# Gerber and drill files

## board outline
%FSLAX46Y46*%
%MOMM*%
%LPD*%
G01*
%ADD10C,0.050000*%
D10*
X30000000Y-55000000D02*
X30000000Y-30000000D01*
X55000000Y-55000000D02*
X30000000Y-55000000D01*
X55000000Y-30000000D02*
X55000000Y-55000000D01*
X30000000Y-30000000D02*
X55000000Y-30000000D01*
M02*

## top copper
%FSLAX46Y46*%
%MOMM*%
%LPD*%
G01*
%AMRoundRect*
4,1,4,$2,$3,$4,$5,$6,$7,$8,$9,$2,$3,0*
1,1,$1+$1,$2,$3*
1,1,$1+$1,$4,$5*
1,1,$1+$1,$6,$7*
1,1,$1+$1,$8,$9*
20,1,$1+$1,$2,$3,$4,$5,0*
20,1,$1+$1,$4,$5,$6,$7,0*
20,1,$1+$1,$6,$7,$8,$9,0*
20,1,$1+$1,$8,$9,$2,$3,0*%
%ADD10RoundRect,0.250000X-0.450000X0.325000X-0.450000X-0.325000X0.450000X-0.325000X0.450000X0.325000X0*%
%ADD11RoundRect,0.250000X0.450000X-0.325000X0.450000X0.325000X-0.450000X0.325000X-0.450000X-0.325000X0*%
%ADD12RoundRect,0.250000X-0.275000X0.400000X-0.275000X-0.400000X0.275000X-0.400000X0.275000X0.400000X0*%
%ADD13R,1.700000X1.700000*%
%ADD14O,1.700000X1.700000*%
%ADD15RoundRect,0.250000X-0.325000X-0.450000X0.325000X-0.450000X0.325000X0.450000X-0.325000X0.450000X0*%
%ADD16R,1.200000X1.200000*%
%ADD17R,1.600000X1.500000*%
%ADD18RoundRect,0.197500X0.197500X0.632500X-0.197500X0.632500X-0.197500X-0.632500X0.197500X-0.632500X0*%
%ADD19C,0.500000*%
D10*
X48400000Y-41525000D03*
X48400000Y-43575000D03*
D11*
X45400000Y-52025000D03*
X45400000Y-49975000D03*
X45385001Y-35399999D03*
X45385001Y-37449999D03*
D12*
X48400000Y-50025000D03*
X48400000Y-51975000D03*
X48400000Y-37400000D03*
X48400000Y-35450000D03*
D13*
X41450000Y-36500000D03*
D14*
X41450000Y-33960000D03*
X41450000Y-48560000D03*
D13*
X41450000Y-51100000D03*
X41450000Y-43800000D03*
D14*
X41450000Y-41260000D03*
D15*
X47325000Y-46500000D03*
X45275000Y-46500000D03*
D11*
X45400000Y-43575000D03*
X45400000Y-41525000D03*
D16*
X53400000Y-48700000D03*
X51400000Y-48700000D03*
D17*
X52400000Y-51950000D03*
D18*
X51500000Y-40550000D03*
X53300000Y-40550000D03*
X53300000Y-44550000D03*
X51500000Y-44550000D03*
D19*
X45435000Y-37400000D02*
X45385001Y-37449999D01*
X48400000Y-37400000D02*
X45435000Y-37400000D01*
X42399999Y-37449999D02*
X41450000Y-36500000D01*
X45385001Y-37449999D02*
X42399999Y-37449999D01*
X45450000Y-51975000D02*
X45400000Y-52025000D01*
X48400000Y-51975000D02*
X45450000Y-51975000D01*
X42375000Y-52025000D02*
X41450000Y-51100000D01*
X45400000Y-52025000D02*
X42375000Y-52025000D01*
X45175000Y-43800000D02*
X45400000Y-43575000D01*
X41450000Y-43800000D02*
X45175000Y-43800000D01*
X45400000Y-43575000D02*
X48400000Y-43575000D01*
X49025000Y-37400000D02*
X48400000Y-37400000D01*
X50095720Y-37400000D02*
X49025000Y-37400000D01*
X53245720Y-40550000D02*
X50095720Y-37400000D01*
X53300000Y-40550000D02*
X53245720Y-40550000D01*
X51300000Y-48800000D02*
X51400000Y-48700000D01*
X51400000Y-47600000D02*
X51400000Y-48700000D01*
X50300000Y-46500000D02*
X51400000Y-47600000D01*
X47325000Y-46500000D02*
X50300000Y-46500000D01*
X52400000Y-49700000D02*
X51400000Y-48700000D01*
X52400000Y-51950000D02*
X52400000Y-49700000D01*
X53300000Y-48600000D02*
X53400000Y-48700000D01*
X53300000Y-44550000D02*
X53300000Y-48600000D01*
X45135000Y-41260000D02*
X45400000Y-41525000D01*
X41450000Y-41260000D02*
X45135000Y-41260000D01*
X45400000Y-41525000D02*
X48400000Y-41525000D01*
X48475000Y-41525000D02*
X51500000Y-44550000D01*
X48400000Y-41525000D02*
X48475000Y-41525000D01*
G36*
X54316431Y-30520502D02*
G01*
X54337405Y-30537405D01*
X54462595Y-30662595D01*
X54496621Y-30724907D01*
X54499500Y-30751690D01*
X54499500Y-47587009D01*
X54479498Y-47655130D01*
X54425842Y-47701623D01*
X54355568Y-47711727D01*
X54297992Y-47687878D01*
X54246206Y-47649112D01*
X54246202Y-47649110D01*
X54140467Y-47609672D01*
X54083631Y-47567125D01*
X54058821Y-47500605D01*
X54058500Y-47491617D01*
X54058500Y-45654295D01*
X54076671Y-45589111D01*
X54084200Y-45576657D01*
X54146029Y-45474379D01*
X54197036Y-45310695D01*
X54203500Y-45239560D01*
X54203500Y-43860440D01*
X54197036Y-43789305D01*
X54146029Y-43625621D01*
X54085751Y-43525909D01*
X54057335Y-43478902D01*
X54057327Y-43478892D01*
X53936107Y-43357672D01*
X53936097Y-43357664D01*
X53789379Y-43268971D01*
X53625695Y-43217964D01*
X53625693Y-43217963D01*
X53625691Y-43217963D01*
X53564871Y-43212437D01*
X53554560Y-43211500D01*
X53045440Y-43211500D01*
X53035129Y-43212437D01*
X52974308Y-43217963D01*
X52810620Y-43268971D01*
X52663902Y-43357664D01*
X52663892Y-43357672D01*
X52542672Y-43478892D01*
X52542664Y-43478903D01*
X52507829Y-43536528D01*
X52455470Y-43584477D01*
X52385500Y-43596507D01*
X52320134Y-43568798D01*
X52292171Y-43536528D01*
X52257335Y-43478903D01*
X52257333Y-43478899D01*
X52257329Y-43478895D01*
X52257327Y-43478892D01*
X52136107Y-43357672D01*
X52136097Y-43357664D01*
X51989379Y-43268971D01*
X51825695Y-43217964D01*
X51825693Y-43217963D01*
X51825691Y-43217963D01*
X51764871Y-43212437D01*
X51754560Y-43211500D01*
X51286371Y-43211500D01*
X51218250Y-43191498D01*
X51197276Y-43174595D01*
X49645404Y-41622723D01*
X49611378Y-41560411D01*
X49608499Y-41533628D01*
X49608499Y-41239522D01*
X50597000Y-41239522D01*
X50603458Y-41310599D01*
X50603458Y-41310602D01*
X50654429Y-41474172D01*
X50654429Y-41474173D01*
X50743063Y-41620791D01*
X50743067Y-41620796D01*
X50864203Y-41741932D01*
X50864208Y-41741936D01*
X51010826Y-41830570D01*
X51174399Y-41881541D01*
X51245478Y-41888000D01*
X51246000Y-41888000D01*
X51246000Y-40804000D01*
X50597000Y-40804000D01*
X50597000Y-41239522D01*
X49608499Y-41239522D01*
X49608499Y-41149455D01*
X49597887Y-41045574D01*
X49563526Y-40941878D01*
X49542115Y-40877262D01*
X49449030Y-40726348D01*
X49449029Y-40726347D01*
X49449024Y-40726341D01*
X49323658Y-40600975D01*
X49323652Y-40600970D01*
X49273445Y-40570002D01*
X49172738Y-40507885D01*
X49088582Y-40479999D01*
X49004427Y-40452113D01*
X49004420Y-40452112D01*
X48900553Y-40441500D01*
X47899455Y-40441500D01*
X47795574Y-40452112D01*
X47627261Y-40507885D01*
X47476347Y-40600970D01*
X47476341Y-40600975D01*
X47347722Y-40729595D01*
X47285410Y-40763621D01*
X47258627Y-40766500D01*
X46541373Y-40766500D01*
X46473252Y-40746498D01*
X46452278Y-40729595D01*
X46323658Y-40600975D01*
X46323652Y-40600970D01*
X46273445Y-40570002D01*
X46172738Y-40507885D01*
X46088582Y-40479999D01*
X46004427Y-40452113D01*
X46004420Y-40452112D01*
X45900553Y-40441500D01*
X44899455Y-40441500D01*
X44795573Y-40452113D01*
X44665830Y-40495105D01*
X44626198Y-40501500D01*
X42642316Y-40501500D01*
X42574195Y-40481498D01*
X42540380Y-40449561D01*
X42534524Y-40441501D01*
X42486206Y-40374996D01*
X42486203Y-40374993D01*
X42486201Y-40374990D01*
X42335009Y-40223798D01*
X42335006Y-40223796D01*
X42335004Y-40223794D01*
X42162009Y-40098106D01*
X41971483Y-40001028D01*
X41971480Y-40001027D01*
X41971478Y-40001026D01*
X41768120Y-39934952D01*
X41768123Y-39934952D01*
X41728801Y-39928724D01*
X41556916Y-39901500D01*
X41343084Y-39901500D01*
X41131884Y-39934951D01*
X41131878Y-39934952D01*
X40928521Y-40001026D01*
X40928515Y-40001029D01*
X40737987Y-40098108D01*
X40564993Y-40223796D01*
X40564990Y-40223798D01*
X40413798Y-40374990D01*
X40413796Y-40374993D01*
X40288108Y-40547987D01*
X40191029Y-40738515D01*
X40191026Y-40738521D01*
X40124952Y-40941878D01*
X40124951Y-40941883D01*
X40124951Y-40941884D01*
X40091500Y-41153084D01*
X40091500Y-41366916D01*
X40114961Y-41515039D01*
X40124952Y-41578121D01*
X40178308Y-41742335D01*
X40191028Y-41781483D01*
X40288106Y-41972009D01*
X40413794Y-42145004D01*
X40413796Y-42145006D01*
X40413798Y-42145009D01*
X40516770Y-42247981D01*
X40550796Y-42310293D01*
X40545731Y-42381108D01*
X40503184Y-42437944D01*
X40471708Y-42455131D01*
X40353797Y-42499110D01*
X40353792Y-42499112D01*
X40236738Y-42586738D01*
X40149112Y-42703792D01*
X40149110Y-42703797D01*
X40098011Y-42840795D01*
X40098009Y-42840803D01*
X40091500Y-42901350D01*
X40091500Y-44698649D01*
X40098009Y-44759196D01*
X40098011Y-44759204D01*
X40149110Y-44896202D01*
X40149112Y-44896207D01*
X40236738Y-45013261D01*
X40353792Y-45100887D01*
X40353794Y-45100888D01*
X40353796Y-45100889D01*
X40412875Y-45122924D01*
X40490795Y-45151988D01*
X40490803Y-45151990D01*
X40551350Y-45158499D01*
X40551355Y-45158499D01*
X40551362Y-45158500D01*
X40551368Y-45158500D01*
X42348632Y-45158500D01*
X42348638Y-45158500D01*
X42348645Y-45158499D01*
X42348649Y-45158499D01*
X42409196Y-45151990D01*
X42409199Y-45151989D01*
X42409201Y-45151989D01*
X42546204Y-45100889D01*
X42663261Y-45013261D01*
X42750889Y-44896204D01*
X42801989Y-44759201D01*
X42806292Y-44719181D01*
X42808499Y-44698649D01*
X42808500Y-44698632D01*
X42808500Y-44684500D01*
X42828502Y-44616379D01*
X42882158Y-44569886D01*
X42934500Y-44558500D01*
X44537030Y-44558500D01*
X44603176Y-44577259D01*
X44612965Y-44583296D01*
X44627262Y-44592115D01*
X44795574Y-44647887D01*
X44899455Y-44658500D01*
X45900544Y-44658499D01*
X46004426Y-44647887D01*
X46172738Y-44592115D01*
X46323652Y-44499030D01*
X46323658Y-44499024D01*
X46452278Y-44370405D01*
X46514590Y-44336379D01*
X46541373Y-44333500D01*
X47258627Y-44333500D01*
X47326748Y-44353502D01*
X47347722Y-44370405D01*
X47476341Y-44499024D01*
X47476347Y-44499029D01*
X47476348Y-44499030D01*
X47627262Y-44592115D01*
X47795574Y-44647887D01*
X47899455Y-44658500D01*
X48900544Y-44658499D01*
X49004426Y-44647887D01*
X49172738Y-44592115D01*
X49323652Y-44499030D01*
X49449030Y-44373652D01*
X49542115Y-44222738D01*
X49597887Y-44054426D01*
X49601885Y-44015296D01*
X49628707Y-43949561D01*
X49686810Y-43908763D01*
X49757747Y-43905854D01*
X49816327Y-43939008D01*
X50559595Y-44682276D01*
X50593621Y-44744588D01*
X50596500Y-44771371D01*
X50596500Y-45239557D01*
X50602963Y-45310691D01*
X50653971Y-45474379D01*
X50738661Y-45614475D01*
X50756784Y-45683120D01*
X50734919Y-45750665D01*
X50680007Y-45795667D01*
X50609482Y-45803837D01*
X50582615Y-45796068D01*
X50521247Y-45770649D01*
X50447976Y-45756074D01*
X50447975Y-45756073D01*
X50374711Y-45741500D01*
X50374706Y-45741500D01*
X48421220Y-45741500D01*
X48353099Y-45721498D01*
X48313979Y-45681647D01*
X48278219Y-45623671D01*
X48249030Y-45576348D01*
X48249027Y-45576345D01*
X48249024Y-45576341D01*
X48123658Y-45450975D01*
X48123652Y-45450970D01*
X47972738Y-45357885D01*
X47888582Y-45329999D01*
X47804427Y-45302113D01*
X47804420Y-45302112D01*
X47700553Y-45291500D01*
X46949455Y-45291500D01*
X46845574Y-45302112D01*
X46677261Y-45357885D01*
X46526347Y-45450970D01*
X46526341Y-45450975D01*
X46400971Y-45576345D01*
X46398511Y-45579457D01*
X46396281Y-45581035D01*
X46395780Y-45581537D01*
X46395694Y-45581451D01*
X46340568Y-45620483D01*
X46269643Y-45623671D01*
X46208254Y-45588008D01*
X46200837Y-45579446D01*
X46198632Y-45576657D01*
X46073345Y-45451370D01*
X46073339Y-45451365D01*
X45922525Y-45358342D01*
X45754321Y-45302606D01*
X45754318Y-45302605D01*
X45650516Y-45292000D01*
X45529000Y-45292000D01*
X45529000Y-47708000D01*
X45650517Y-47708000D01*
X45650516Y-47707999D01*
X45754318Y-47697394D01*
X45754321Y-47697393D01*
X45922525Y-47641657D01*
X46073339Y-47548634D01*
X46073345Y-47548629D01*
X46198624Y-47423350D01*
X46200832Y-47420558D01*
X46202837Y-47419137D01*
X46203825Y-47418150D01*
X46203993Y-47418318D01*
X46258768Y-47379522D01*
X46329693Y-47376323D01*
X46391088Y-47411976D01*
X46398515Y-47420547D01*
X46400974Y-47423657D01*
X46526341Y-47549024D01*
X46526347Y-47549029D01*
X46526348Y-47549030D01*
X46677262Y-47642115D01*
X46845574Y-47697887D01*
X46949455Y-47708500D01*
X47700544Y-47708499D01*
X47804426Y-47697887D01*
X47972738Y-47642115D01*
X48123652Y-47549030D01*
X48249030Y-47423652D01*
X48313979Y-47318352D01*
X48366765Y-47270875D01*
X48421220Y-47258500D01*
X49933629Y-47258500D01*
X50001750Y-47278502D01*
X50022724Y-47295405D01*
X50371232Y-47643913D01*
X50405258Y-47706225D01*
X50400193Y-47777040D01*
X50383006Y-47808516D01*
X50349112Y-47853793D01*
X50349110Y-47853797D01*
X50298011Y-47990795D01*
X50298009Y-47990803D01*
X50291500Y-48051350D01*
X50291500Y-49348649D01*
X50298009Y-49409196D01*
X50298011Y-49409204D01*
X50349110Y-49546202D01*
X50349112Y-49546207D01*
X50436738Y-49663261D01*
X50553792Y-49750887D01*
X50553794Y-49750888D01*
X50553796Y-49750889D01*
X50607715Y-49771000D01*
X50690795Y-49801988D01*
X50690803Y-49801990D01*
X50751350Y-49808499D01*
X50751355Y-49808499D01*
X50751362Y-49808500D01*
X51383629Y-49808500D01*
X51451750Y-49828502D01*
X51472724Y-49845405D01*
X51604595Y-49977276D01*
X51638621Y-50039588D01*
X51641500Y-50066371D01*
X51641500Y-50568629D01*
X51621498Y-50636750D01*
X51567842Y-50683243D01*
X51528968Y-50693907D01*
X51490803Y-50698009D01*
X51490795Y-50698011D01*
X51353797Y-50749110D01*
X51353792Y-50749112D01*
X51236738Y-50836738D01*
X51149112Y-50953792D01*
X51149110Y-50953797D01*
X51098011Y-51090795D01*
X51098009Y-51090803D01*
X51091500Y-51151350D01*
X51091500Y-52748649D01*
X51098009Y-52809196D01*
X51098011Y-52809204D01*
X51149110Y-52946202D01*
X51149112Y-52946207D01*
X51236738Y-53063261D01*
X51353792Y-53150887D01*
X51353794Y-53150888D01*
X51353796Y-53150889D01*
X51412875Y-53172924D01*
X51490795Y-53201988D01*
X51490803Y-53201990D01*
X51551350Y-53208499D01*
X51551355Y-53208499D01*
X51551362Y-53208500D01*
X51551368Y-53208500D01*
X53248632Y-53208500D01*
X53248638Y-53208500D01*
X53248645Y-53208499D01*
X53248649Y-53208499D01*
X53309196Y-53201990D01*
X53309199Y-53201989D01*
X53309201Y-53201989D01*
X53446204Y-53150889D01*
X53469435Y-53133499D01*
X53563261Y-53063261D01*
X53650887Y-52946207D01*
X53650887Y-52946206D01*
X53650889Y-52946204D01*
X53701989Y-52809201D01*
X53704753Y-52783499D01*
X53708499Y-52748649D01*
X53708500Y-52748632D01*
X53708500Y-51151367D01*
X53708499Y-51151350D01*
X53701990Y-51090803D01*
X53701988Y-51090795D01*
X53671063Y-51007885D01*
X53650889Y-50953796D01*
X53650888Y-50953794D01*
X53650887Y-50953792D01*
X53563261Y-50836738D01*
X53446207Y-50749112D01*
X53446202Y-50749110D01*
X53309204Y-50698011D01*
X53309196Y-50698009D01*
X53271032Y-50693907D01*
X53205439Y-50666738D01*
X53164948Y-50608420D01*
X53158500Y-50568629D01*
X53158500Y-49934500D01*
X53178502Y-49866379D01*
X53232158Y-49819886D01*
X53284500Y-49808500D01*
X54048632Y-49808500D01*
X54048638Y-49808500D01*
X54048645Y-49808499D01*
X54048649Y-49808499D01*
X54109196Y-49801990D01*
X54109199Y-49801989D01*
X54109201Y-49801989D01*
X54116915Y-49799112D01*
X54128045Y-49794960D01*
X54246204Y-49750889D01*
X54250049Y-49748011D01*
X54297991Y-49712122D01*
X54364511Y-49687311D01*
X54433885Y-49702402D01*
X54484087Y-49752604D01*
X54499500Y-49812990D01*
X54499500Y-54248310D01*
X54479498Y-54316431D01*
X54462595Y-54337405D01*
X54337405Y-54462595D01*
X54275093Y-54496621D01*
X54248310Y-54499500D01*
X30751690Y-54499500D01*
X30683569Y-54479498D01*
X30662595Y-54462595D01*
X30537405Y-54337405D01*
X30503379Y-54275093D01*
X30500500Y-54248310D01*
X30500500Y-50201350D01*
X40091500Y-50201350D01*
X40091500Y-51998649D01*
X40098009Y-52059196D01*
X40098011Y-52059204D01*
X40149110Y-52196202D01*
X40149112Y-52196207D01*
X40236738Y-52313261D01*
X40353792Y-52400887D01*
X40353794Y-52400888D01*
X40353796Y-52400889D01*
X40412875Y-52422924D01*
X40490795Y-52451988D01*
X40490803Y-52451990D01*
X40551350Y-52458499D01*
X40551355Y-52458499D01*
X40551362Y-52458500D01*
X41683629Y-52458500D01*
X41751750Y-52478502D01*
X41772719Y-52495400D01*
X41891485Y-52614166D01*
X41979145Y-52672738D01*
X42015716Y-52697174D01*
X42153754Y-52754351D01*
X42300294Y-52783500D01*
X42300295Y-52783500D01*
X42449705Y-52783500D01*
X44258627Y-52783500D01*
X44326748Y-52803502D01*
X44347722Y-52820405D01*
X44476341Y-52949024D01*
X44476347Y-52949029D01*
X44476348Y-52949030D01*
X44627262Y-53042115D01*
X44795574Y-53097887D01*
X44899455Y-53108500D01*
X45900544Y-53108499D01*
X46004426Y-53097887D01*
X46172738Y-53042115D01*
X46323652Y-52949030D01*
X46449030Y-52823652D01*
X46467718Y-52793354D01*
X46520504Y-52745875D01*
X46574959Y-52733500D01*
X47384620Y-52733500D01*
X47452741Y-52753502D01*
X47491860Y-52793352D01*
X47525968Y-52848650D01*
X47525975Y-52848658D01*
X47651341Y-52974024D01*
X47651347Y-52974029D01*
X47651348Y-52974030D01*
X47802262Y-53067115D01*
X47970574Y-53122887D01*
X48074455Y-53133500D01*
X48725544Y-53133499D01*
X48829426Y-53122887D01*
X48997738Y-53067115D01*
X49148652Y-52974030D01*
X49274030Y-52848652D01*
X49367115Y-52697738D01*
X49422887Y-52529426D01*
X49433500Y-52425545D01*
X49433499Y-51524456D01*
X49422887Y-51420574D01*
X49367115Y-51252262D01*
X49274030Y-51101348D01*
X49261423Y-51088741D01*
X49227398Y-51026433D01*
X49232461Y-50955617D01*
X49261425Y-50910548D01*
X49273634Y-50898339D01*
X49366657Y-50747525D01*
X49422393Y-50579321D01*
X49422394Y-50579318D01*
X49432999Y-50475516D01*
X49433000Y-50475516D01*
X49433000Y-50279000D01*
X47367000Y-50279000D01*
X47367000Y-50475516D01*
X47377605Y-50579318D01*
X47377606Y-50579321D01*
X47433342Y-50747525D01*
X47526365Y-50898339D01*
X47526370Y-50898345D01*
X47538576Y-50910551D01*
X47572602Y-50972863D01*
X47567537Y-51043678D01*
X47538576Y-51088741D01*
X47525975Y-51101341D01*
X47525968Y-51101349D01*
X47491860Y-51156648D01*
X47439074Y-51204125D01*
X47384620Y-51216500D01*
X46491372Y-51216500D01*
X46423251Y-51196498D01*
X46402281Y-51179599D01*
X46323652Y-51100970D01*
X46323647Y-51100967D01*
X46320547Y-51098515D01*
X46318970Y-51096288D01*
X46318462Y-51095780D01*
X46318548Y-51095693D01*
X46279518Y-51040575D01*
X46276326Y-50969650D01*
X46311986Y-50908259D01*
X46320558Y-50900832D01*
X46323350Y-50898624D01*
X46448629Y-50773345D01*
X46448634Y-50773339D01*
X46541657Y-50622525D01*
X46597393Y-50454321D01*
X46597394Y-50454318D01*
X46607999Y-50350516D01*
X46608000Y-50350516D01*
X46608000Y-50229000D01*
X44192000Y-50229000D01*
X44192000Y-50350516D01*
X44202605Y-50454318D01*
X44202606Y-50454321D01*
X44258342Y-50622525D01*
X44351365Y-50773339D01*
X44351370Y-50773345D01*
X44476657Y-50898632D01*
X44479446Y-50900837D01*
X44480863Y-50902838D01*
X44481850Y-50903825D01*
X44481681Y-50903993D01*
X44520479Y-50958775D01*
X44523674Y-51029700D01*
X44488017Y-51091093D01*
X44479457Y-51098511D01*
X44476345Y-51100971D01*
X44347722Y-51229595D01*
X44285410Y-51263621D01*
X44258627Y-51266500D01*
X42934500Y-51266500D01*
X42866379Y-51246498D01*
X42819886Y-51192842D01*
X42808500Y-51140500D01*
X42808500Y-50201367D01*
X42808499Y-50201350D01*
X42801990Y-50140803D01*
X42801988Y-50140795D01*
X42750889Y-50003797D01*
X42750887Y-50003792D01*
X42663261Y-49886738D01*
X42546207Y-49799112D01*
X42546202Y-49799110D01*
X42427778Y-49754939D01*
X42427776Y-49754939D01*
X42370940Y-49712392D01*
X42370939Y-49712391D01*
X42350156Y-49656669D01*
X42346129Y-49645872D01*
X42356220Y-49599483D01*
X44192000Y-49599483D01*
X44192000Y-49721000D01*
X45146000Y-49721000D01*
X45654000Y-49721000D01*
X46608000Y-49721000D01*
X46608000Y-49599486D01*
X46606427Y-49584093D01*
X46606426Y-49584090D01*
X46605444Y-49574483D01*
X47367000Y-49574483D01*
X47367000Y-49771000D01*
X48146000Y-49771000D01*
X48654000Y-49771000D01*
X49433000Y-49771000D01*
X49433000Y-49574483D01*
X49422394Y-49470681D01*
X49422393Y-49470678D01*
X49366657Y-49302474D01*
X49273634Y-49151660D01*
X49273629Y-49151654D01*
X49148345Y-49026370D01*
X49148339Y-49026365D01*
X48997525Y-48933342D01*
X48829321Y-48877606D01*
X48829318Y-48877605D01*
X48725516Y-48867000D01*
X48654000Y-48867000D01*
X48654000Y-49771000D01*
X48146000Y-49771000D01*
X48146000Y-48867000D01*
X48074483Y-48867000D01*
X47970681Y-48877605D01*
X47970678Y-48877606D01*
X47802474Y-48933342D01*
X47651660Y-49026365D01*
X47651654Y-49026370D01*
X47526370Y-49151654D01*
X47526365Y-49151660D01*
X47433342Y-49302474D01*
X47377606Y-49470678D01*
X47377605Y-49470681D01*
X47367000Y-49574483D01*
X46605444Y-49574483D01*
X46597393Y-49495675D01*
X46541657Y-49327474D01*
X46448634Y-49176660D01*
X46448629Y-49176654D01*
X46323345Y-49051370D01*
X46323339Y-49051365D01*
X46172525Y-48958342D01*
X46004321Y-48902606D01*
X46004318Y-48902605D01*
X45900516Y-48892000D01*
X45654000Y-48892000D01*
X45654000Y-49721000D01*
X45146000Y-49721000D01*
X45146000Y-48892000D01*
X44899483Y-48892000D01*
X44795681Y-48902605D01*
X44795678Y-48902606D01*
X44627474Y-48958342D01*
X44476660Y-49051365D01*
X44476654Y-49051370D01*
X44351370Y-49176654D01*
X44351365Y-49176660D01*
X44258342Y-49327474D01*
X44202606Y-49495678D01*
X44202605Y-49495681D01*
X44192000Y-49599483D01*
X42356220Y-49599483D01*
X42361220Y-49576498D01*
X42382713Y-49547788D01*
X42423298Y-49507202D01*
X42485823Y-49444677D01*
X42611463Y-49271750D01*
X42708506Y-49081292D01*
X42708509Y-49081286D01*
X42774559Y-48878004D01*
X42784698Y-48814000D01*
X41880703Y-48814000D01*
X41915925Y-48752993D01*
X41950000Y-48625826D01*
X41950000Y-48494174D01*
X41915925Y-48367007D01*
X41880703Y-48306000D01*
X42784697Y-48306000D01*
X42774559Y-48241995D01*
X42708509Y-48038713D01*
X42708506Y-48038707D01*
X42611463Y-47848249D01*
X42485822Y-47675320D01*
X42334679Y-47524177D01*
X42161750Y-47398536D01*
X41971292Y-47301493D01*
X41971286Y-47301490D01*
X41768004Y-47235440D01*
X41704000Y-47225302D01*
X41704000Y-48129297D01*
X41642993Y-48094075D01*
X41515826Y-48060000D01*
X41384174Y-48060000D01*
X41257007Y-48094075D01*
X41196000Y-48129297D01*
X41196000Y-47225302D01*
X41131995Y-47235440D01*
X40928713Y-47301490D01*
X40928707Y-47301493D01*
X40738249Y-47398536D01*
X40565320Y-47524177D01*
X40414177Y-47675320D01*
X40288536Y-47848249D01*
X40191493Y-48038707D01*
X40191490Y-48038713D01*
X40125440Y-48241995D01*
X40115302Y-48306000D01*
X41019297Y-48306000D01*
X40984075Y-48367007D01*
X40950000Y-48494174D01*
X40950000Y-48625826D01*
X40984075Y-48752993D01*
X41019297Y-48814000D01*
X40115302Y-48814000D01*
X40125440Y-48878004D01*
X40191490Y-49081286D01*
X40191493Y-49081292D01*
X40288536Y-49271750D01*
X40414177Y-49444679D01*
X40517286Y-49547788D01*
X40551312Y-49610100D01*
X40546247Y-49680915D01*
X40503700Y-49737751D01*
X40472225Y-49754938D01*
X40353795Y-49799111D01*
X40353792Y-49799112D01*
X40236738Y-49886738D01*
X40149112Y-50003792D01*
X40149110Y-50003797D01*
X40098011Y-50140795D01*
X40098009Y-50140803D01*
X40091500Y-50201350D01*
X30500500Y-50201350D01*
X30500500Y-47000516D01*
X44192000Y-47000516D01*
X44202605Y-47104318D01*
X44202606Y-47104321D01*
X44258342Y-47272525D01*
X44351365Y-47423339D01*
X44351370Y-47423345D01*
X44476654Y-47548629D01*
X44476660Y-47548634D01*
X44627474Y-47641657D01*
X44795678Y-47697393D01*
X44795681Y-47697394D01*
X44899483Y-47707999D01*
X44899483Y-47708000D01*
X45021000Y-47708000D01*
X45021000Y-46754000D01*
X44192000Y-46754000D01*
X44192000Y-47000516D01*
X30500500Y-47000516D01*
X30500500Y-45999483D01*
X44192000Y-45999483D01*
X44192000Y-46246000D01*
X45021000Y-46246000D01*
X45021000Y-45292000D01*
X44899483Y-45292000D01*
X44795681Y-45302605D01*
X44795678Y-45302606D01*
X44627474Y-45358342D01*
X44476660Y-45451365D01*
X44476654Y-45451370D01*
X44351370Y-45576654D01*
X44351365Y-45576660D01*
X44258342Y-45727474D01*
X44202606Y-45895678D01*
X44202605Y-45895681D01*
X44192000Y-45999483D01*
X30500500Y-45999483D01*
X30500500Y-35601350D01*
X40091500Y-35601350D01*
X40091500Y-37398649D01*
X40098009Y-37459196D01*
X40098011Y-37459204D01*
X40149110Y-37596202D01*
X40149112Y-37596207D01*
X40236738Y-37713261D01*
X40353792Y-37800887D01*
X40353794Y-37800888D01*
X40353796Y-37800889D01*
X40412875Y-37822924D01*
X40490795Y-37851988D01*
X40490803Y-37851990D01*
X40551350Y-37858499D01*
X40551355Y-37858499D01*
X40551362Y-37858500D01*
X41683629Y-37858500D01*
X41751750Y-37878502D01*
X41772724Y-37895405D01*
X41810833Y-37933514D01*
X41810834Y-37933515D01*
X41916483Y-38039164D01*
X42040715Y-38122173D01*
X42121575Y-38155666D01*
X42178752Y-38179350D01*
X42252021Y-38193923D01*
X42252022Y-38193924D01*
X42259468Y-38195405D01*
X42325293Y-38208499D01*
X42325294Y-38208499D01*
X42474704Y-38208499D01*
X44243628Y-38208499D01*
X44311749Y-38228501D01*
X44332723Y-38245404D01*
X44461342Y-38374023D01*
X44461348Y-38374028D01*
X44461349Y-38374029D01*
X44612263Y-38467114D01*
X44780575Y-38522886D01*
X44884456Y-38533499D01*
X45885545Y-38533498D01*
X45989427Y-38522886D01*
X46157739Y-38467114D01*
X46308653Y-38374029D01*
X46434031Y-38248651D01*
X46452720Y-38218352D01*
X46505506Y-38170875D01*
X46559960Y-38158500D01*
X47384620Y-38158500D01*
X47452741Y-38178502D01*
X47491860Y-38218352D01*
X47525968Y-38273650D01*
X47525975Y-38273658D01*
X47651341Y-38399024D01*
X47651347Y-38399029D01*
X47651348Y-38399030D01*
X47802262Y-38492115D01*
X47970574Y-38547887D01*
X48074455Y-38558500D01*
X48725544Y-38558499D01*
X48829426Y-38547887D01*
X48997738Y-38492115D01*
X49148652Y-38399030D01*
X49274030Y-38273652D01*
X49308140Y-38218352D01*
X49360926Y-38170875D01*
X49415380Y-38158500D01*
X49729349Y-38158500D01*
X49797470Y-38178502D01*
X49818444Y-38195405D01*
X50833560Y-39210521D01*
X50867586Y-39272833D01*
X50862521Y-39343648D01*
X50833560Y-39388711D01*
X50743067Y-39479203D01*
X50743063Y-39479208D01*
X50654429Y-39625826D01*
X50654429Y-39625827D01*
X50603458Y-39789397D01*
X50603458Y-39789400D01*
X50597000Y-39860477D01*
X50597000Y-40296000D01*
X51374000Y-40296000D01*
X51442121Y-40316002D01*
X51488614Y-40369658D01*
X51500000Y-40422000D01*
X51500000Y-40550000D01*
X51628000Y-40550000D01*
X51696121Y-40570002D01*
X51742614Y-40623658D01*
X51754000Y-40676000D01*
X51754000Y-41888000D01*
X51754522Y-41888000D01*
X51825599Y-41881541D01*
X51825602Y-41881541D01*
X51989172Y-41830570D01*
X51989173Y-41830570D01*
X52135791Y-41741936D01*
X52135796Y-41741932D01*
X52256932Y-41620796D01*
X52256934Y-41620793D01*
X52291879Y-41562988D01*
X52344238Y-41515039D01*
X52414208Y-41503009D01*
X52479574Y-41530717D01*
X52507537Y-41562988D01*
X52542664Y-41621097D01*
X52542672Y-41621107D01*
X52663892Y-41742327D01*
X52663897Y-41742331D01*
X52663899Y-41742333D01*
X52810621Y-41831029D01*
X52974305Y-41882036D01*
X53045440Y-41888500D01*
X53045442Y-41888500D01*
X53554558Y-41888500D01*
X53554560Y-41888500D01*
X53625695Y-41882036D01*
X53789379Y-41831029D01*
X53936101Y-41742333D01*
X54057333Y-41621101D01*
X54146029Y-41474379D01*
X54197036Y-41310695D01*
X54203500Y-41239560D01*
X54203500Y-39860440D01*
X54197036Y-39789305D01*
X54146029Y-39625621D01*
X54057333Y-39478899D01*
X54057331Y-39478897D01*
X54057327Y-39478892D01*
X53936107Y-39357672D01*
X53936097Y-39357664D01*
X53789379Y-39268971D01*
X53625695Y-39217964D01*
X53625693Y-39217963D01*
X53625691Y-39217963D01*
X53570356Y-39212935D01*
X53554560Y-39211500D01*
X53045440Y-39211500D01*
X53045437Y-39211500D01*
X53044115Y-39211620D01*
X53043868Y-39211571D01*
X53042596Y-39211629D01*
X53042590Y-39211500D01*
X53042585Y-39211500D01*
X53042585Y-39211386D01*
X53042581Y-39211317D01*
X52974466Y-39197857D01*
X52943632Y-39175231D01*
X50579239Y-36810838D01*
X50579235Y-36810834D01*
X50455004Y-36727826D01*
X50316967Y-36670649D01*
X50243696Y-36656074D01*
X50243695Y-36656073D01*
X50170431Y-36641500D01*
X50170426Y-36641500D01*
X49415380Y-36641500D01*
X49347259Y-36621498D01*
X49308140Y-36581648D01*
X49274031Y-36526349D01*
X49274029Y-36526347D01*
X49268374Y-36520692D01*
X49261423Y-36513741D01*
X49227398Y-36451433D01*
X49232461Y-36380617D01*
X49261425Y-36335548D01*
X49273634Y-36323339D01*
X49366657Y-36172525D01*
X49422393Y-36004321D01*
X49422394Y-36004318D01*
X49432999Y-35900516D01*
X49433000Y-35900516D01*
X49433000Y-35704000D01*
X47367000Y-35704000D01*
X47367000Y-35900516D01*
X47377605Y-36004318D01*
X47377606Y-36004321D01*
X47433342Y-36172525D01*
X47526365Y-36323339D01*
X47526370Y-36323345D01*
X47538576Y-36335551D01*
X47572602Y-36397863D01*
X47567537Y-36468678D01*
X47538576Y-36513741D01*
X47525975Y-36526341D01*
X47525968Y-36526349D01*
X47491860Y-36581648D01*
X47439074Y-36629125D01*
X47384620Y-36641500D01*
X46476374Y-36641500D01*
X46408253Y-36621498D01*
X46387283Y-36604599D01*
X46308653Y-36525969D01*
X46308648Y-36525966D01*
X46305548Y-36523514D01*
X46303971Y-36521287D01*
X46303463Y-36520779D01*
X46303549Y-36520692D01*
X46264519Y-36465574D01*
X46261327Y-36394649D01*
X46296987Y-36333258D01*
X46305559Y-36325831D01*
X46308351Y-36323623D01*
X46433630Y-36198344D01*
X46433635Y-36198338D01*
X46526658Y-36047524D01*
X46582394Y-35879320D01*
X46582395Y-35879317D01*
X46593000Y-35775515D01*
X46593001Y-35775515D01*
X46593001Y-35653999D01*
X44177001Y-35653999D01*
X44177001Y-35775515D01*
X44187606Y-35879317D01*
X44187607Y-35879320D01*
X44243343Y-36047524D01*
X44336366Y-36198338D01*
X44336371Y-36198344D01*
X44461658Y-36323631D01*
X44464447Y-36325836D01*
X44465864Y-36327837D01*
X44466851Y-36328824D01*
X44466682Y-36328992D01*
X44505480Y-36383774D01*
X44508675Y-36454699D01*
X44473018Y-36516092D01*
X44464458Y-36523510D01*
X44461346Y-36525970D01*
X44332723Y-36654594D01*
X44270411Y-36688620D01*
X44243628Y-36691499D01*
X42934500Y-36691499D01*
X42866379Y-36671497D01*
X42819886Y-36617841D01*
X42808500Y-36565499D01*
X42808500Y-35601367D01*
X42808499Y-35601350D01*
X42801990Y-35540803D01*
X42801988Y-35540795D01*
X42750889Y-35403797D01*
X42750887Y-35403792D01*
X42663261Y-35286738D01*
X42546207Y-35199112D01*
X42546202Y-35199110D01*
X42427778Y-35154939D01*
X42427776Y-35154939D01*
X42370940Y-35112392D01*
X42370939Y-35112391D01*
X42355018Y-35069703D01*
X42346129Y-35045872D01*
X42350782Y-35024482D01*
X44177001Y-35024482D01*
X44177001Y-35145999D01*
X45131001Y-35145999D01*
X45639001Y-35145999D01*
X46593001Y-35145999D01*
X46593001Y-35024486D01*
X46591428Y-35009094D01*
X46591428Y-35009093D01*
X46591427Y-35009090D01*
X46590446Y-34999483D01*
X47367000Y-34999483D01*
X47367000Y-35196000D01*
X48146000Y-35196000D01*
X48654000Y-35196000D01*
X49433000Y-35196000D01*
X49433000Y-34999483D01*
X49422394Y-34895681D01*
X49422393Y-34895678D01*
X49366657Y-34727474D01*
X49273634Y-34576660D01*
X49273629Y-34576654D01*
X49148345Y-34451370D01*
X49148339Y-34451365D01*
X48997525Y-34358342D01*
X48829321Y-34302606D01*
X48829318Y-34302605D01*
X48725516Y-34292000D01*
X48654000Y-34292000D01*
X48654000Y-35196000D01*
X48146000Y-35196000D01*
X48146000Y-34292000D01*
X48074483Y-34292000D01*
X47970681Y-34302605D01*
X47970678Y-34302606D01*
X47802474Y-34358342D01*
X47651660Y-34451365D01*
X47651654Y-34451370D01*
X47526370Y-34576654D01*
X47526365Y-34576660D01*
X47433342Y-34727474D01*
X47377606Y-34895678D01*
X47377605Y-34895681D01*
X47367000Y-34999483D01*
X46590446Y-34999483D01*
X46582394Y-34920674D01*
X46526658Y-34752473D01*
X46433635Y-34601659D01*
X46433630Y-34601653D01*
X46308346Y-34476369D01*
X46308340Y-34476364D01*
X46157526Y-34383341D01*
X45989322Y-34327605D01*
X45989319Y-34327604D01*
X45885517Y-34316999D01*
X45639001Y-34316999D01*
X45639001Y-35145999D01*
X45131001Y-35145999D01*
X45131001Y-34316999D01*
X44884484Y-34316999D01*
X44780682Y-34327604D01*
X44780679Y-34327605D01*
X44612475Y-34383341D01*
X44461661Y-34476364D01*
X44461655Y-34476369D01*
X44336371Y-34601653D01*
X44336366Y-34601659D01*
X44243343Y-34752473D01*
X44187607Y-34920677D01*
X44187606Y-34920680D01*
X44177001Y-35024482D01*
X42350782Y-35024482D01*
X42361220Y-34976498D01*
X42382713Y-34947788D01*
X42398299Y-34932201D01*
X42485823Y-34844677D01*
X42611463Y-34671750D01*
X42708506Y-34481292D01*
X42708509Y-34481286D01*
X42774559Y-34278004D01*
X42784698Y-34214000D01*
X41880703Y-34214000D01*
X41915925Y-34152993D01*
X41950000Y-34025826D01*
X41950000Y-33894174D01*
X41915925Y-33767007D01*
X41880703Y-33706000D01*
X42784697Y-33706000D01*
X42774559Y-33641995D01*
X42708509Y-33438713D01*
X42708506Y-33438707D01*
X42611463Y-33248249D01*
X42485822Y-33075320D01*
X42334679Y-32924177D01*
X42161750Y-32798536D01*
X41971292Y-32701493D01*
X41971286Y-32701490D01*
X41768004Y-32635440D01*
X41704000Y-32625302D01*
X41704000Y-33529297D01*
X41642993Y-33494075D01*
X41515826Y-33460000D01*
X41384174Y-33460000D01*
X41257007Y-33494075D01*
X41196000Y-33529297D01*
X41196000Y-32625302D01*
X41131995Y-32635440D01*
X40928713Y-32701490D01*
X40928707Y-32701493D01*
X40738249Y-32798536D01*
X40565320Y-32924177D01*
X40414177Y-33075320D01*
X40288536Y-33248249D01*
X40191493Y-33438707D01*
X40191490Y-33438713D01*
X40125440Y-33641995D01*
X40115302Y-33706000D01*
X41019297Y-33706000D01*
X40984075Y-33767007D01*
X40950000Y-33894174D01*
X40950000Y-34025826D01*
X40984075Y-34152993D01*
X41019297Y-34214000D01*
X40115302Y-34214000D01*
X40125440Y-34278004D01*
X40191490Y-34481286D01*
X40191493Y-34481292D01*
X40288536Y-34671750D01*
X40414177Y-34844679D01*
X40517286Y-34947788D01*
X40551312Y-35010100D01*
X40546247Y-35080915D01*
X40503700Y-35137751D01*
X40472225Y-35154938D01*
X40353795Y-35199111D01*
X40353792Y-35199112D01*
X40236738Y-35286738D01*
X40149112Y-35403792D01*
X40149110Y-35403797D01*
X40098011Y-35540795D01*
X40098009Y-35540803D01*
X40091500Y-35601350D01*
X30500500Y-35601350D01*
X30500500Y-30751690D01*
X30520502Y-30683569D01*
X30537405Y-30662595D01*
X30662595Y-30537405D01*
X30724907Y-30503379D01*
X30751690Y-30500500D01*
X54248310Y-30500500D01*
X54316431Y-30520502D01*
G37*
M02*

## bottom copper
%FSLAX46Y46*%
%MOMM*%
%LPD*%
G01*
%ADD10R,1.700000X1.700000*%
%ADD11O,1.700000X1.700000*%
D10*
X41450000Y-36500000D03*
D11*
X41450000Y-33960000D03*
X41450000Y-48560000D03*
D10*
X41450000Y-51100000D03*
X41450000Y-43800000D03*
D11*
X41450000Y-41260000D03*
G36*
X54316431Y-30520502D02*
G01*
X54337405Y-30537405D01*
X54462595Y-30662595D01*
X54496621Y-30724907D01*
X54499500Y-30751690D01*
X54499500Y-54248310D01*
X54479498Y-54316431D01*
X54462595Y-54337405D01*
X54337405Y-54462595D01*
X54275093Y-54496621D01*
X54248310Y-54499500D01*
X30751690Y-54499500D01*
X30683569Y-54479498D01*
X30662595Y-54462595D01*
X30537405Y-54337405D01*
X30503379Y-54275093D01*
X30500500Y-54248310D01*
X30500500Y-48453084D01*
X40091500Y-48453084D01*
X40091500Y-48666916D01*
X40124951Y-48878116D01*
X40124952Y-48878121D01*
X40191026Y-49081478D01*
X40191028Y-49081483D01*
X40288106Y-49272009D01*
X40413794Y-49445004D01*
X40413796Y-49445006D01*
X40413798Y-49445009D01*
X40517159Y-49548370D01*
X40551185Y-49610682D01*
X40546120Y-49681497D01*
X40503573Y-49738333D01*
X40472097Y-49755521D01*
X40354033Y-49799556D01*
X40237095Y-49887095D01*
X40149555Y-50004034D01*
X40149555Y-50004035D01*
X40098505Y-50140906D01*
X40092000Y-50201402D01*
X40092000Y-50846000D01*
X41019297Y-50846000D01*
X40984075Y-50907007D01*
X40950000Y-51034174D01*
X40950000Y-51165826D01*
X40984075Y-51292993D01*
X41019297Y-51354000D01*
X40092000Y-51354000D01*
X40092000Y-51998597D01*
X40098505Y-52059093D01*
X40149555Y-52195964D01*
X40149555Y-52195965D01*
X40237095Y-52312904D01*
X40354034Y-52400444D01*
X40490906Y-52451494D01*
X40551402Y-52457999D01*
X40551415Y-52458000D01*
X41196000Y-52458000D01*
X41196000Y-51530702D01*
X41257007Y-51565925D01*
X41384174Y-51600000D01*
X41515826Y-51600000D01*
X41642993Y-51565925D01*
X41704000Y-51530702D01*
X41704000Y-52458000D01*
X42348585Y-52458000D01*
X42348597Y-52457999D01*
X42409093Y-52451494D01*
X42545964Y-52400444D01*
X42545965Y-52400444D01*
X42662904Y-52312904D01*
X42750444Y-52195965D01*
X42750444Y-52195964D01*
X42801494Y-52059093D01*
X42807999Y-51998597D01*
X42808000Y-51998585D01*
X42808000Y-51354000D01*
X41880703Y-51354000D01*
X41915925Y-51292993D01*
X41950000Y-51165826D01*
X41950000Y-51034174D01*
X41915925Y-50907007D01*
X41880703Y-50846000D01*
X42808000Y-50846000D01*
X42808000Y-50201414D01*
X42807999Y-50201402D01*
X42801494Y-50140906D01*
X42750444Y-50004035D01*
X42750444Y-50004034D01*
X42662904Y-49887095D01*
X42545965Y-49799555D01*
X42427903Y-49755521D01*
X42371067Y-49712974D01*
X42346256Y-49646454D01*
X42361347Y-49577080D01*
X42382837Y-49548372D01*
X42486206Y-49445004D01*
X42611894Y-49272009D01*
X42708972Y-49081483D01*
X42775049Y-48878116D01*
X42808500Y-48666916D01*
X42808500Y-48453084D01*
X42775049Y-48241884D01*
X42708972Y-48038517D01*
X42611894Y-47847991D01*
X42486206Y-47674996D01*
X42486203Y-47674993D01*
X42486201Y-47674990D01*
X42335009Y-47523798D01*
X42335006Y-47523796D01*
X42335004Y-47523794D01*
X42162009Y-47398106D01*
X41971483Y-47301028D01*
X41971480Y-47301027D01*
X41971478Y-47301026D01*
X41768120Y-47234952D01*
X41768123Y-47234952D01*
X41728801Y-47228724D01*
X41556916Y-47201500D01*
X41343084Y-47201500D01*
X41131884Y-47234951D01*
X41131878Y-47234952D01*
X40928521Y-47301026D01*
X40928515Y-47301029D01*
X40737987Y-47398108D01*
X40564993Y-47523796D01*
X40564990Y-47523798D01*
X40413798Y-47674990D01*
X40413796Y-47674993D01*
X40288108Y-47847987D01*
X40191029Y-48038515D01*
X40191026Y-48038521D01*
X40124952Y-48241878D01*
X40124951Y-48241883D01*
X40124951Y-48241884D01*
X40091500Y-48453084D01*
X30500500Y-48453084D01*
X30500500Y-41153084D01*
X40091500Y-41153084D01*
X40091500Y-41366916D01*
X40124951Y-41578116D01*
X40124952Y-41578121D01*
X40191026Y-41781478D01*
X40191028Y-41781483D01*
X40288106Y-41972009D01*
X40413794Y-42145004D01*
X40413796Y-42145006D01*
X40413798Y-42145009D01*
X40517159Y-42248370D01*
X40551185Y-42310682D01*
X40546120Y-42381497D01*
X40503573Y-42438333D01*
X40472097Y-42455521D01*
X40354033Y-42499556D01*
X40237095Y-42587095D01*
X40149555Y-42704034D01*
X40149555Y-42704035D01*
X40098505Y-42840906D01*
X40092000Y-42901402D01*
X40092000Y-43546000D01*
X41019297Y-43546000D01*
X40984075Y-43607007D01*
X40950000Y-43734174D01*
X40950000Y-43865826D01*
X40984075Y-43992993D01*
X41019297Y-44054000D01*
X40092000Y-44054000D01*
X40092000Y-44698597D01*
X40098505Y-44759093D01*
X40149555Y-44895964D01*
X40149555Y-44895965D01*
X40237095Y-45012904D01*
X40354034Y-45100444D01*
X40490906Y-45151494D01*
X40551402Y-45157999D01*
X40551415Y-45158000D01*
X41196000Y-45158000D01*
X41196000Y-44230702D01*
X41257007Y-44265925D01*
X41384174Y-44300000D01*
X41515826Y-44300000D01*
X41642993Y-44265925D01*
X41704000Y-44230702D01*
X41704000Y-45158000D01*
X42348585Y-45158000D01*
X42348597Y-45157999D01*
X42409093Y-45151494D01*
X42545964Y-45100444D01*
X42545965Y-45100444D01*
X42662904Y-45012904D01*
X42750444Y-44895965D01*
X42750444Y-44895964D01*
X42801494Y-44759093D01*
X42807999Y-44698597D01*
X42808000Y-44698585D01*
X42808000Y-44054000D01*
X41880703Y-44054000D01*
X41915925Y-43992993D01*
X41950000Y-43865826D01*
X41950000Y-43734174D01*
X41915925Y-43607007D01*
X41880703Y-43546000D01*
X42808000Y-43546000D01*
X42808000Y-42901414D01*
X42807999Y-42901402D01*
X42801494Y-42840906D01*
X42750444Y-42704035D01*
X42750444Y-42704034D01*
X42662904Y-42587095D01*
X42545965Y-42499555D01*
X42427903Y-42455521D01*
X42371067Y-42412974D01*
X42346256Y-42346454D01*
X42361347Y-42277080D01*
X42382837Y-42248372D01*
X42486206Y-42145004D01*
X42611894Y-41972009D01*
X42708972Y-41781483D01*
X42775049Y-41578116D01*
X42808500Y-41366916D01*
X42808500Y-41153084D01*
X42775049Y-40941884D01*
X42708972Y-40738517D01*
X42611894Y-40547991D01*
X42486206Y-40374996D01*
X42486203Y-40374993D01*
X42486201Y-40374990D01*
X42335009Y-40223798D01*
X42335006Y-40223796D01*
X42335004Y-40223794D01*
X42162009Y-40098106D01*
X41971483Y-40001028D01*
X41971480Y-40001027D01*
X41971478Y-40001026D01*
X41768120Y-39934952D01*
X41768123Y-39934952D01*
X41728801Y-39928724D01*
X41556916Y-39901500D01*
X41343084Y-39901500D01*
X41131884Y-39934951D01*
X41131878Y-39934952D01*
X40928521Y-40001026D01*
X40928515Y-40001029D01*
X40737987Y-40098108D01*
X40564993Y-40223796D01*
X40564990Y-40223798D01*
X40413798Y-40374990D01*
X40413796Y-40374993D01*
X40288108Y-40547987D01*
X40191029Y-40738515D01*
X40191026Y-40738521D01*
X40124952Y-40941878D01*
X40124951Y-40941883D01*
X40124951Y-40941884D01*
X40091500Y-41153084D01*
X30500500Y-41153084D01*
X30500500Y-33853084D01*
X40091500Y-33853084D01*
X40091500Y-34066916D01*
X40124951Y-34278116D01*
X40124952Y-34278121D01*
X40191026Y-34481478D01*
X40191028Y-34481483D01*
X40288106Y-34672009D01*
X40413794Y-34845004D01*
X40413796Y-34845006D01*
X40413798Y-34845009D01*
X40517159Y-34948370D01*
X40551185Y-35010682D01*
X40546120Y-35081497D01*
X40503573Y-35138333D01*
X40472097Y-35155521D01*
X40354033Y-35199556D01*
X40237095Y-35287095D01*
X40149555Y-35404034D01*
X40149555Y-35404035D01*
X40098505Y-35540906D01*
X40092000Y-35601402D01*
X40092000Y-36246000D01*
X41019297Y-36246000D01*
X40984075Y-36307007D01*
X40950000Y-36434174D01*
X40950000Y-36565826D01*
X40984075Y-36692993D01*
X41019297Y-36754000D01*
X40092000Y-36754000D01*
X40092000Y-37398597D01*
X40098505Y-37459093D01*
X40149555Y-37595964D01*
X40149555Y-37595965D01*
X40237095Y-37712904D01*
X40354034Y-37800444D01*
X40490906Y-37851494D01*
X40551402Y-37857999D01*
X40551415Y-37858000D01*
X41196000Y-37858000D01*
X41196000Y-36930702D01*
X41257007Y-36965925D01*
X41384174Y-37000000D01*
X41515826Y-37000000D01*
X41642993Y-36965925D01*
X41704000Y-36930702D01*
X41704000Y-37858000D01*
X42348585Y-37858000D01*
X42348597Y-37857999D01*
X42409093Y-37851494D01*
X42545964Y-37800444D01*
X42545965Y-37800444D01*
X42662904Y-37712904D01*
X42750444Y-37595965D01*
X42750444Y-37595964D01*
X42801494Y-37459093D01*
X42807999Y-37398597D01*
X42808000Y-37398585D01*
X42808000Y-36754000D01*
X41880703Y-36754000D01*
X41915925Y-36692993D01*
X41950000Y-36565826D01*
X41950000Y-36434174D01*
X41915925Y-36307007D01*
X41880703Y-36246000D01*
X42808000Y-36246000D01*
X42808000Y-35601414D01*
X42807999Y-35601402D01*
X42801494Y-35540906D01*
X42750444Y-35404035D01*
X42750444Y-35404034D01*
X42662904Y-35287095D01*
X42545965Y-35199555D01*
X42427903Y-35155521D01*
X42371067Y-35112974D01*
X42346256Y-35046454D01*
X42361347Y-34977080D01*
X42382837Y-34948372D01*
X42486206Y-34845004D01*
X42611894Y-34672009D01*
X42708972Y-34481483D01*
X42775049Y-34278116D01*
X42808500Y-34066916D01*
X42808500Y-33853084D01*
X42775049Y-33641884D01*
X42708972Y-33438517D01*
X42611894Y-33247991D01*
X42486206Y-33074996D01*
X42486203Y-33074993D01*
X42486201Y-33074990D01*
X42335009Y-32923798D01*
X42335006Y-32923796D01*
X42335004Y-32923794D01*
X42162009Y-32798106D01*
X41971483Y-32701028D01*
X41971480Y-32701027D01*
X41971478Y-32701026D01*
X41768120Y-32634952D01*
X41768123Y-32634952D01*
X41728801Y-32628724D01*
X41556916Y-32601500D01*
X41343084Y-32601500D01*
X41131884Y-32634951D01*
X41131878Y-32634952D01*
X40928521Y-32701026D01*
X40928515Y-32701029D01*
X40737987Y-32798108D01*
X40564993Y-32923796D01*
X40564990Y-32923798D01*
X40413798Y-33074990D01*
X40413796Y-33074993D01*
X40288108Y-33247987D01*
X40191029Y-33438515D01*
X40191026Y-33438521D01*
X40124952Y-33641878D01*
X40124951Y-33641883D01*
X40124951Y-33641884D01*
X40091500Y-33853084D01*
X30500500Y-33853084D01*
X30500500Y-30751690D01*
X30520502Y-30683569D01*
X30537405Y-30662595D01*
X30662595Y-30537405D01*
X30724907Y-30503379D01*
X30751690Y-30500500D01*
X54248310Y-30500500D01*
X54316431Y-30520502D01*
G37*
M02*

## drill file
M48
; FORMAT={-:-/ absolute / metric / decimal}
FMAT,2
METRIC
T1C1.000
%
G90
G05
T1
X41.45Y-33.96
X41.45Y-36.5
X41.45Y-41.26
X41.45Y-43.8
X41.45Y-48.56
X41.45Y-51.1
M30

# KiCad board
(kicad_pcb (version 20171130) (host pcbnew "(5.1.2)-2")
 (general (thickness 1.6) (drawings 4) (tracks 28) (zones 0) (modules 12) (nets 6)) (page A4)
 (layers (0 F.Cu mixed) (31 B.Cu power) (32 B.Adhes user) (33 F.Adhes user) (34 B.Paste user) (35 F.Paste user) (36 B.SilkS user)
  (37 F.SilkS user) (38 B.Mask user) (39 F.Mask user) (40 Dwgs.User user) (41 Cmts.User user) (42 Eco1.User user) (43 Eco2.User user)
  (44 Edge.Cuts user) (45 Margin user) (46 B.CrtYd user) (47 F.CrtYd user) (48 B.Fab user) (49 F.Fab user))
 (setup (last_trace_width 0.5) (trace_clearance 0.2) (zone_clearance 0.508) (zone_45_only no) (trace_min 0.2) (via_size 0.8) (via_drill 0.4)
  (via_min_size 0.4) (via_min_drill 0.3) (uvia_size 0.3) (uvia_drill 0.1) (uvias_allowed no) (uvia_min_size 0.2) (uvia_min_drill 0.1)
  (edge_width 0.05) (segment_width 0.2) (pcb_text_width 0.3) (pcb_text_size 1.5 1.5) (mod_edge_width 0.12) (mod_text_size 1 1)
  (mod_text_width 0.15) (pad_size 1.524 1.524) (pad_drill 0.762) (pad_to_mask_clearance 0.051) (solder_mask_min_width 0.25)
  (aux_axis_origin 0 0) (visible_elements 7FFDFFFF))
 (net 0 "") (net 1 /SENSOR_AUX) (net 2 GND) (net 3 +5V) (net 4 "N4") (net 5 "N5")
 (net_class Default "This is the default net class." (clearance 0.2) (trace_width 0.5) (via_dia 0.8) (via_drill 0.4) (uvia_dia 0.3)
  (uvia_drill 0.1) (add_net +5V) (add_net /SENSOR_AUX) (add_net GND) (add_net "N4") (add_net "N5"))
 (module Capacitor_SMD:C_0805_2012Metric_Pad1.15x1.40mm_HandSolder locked (layer F.Cu) (at 48.4 42.55 270)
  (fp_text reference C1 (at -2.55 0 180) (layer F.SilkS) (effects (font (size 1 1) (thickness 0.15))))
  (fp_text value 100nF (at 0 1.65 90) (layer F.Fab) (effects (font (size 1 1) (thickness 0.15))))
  (pad 1 smd roundrect (at -1.025 0 270) (size 1.15 1.4) (layers F.Cu F.Paste F.Mask) (roundrect_rratio 0.217391) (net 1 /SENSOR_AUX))
  (pad 2 smd roundrect (at 1.025 0 270) (size 1.15 1.4) (layers F.Cu F.Paste F.Mask) (roundrect_rratio 0.217391) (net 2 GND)))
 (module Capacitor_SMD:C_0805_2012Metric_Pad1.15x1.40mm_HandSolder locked (layer F.Cu) (at 45.4 51 90)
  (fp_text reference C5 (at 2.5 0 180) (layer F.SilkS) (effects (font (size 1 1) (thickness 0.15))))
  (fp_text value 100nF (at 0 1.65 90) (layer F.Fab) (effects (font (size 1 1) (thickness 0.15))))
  (pad 1 smd roundrect (at -1.025 0 90) (size 1.15 1.4) (layers F.Cu F.Paste F.Mask) (roundrect_rratio 0.217391) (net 2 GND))
  (pad 2 smd roundrect (at 1.025 0 90) (size 1.15 1.4) (layers F.Cu F.Paste F.Mask) (roundrect_rratio 0.217391) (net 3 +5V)))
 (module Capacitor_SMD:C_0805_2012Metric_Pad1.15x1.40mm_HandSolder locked (layer F.Cu) (at 45.385001 36.424999 90)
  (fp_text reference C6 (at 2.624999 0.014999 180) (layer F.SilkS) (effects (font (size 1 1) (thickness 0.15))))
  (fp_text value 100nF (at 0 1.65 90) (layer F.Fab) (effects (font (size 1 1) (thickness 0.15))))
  (pad 2 smd roundrect (at 1.025 0 90) (size 1.15 1.4) (layers F.Cu F.Paste F.Mask) (roundrect_rratio 0.217391) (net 3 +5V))
  (pad 1 smd roundrect (at -1.025 0 90) (size 1.15 1.4) (layers F.Cu F.Paste F.Mask) (roundrect_rratio 0.217391) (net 2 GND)))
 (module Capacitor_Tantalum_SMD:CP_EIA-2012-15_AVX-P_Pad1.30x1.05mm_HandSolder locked (layer F.Cu) (at 48.4 51 270)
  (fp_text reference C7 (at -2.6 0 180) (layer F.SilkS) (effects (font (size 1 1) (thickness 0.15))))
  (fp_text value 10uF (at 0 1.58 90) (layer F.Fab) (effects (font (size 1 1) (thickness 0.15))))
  (pad 1 smd roundrect (at -0.975 0 270) (size 1.3 1.05) (layers F.Cu F.Paste F.Mask) (roundrect_rratio 0.238095) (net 3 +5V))
  (pad 2 smd roundrect (at 0.975 0 270) (size 1.3 1.05) (layers F.Cu F.Paste F.Mask) (roundrect_rratio 0.238095) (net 2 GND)))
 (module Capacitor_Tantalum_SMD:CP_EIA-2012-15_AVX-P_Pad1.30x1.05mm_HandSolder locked (layer F.Cu) (at 48.4 36.425 270)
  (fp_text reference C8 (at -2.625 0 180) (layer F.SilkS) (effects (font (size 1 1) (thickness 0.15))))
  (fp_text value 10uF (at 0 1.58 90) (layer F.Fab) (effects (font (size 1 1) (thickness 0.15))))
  (pad 2 smd roundrect (at 0.975 0 270) (size 1.3 1.05) (layers F.Cu F.Paste F.Mask) (roundrect_rratio 0.238095) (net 2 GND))
  (pad 1 smd roundrect (at -0.975 0 270) (size 1.3 1.05) (layers F.Cu F.Paste F.Mask) (roundrect_rratio 0.238095) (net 3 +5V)))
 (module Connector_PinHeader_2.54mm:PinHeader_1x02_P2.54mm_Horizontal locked (layer F.Cu) (at 41.45 36.5 180)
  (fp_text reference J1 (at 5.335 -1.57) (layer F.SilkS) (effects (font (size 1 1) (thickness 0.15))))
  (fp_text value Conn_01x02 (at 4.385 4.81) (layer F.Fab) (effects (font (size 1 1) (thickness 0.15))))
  (pad 1 thru_hole rect (at 0 0 180) (size 1.7 1.7) (drill 1) (layers *.Cu *.Mask) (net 2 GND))
  (pad 2 thru_hole oval (at 0 2.54 180) (size 1.7 1.7) (drill 1) (layers *.Cu *.Mask) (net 3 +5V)))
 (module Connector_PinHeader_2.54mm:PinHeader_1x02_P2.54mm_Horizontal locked (layer F.Cu) (at 41.45 51.1 180)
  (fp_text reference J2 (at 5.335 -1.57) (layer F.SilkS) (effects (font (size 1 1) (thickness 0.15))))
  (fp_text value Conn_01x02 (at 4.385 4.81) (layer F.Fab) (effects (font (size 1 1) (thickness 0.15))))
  (pad 2 thru_hole oval (at 0 2.54 180) (size 1.7 1.7) (drill 1) (layers *.Cu *.Mask) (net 3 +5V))
  (pad 1 thru_hole rect (at 0 0 180) (size 1.7 1.7) (drill 1) (layers *.Cu *.Mask) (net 2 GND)))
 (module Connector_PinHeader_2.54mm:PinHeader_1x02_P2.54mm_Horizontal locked (layer F.Cu) (at 41.45 43.8 180)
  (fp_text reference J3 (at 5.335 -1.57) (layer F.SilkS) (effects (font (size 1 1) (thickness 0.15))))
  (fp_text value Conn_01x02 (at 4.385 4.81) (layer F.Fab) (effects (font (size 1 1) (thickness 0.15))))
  (pad 1 thru_hole rect (at 0 0 180) (size 1.7 1.7) (drill 1) (layers *.Cu *.Mask) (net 2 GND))
  (pad 2 thru_hole oval (at 0 2.54 180) (size 1.7 1.7) (drill 1) (layers *.Cu *.Mask) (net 1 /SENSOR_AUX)))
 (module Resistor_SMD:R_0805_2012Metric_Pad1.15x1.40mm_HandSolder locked (layer F.Cu) (at 46.3 46.5)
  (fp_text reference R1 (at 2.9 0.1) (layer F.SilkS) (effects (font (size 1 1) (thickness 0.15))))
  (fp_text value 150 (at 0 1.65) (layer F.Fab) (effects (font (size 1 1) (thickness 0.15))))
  (pad 2 smd roundrect (at 1.025 0) (size 1.15 1.4) (layers F.Cu F.Paste F.Mask) (roundrect_rratio 0.217391) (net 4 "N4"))
  (pad 1 smd roundrect (at -1.025 0) (size 1.15 1.4) (layers F.Cu F.Paste F.Mask) (roundrect_rratio 0.217391) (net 3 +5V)))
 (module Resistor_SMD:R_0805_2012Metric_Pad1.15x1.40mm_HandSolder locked (layer F.Cu) (at 45.4 42.55 90)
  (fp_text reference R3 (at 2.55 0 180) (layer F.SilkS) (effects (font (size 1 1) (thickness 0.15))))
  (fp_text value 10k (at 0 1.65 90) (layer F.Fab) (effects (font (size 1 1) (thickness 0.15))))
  (pad 1 smd roundrect (at -1.025 0 90) (size 1.15 1.4) (layers F.Cu F.Paste F.Mask) (roundrect_rratio 0.217391) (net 2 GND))
  (pad 2 smd roundrect (at 1.025 0 90) (size 1.15 1.4) (layers F.Cu F.Paste F.Mask) (roundrect_rratio 0.217391) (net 1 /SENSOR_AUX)))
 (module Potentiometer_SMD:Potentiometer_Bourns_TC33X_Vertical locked (layer F.Cu) (at 52.4 50.5 270)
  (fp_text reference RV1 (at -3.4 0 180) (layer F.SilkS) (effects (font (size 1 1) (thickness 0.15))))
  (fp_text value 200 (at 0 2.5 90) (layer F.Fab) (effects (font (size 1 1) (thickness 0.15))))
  (pad 1 smd rect (at -1.8 -1 270) (size 1.2 1.2) (layers F.Cu F.Paste F.Mask) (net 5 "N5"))
  (pad 3 smd rect (at -1.8 1 270) (size 1.2 1.2) (layers F.Cu F.Paste F.Mask) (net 4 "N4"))
  (pad 2 smd rect (at 1.45 0 270) (size 1.5 1.6) (layers F.Cu F.Paste F.Mask) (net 4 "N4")))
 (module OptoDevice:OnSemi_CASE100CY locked (layer F.Cu) (at 52.4 42.55 180)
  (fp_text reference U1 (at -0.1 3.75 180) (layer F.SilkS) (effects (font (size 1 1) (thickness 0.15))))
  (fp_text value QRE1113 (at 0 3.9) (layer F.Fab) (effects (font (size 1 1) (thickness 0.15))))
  (pad 3 smd roundrect (at 0.9 2 180) (size 0.79 1.66) (layers F.Cu F.Paste F.Mask) (roundrect_rratio 0.25) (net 3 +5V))
  (pad 2 smd roundrect (at -0.9 2 180) (size 0.79 1.66) (layers F.Cu F.Paste F.Mask) (roundrect_rratio 0.25) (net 2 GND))
  (pad 1 smd roundrect (at -0.9 -2 180) (size 0.79 1.66) (layers F.Cu F.Paste F.Mask) (roundrect_rratio 0.25) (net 5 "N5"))
  (pad 4 smd roundrect (at 0.9 -2 180) (size 0.79 1.66) (layers F.Cu F.Paste F.Mask) (roundrect_rratio 0.25) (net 1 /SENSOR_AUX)))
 (gr_line (start 30 55) (end 30 30) (layer Edge.Cuts) (width 0.05))
 (gr_line (start 55 55) (end 30 55) (layer Edge.Cuts) (width 0.05))
 (gr_line (start 55 30) (end 55 55) (layer Edge.Cuts) (width 0.05))
 (gr_line (start 30 30) (end 55 30) (layer Edge.Cuts) (width 0.05))
 (segment (start 45.435 37.4) (end 45.385001 37.449999) (width 0.5) (layer F.Cu) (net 2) (status 40030))
 (segment (start 48.4 37.4) (end 45.435 37.4) (width 0.5) (layer F.Cu) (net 2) (status 40030))
 (segment (start 42.399999 37.449999) (end 41.45 36.5) (width 0.5) (layer F.Cu) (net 2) (status 40020))
 (segment (start 45.385001 37.449999) (end 42.399999 37.449999) (width 0.5) (layer F.Cu) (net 2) (status 40010))
 (segment (start 45.45 51.975) (end 45.4 52.025) (width 0.5) (layer F.Cu) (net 2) (status 40030))
 (segment (start 48.4 51.975) (end 45.45 51.975) (width 0.5) (layer F.Cu) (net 2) (status 40030))
 (segment (start 42.375 52.025) (end 41.45 51.1) (width 0.5) (layer F.Cu) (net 2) (status 40020))
 (segment (start 45.4 52.025) (end 42.375 52.025) (width 0.5) (layer F.Cu) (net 2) (status 40010))
 (segment (start 45.175 43.8) (end 45.4 43.575) (width 0.5) (layer F.Cu) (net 2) (status 40030))
 (segment (start 41.45 43.8) (end 45.175 43.8) (width 0.5) (layer F.Cu) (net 2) (status 40030))
 (segment (start 45.4 43.575) (end 48.4 43.575) (width 0.5) (layer F.Cu) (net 2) (status 40030))
 (segment (start 49.025 37.4) (end 48.4 37.4) (width 0.5) (layer F.Cu) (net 2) (status 40000))
 (segment (start 50.09572 37.4) (end 49.025 37.4) (width 0.5) (layer F.Cu) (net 2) (status 40000))
 (segment (start 53.24572 40.55) (end 50.09572 37.4) (width 0.5) (layer F.Cu) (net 2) (status 40000))
 (segment (start 53.3 40.55) (end 53.24572 40.55) (width 0.5) (layer F.Cu) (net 2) (status 40000))
 (segment (start 51.3 48.8) (end 51.4 48.7) (width 0.5) (layer F.Cu) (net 4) (status 40030))
 (segment (start 51.4 47.6) (end 51.4 48.7) (width 0.5) (layer F.Cu) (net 4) (status 40000))
 (segment (start 50.3 46.5) (end 51.4 47.6) (width 0.5) (layer F.Cu) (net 4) (status 40000))
 (segment (start 47.325 46.5) (end 50.3 46.5) (width 0.5) (layer F.Cu) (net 4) (status 40000))
 (segment (start 52.4 49.7) (end 51.4 48.7) (width 0.5) (layer F.Cu) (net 4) (status 40000))
 (segment (start 52.4 51.95) (end 52.4 49.7) (width 0.5) (layer F.Cu) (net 4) (status 40000))
 (segment (start 53.3 48.6) (end 53.4 48.7) (width 0.5) (layer F.Cu) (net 5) (status 40000))
 (segment (start 53.3 44.55) (end 53.3 48.6) (width 0.5) (layer F.Cu) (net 5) (status 40000))
 (segment (start 45.135 41.26) (end 45.4 41.525) (width 0.5) (layer F.Cu) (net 1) (status 40030))
 (segment (start 41.45 41.26) (end 45.135 41.26) (width 0.5) (layer F.Cu) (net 1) (status 40030))
 (segment (start 45.4 41.525) (end 48.4 41.525) (width 0.5) (layer F.Cu) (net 1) (status 40030))
 (segment (start 48.475 41.525) (end 51.5 44.55) (width 0.5) (layer F.Cu) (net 1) (status 40000))
 (segment (start 48.4 41.525) (end 48.475 41.525) (width 0.5) (layer F.Cu) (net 1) (status 40000))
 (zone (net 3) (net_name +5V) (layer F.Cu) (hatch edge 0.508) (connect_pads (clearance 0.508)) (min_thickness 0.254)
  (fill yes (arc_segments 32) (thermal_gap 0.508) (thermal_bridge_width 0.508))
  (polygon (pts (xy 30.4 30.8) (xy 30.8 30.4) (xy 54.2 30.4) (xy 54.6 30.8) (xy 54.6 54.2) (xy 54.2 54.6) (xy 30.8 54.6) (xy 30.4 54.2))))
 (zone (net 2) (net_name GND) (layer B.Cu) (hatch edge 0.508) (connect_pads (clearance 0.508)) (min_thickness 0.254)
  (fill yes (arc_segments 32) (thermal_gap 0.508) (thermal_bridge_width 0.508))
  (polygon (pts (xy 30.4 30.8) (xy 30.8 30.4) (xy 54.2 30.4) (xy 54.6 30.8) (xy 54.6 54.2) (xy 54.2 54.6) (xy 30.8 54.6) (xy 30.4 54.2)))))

